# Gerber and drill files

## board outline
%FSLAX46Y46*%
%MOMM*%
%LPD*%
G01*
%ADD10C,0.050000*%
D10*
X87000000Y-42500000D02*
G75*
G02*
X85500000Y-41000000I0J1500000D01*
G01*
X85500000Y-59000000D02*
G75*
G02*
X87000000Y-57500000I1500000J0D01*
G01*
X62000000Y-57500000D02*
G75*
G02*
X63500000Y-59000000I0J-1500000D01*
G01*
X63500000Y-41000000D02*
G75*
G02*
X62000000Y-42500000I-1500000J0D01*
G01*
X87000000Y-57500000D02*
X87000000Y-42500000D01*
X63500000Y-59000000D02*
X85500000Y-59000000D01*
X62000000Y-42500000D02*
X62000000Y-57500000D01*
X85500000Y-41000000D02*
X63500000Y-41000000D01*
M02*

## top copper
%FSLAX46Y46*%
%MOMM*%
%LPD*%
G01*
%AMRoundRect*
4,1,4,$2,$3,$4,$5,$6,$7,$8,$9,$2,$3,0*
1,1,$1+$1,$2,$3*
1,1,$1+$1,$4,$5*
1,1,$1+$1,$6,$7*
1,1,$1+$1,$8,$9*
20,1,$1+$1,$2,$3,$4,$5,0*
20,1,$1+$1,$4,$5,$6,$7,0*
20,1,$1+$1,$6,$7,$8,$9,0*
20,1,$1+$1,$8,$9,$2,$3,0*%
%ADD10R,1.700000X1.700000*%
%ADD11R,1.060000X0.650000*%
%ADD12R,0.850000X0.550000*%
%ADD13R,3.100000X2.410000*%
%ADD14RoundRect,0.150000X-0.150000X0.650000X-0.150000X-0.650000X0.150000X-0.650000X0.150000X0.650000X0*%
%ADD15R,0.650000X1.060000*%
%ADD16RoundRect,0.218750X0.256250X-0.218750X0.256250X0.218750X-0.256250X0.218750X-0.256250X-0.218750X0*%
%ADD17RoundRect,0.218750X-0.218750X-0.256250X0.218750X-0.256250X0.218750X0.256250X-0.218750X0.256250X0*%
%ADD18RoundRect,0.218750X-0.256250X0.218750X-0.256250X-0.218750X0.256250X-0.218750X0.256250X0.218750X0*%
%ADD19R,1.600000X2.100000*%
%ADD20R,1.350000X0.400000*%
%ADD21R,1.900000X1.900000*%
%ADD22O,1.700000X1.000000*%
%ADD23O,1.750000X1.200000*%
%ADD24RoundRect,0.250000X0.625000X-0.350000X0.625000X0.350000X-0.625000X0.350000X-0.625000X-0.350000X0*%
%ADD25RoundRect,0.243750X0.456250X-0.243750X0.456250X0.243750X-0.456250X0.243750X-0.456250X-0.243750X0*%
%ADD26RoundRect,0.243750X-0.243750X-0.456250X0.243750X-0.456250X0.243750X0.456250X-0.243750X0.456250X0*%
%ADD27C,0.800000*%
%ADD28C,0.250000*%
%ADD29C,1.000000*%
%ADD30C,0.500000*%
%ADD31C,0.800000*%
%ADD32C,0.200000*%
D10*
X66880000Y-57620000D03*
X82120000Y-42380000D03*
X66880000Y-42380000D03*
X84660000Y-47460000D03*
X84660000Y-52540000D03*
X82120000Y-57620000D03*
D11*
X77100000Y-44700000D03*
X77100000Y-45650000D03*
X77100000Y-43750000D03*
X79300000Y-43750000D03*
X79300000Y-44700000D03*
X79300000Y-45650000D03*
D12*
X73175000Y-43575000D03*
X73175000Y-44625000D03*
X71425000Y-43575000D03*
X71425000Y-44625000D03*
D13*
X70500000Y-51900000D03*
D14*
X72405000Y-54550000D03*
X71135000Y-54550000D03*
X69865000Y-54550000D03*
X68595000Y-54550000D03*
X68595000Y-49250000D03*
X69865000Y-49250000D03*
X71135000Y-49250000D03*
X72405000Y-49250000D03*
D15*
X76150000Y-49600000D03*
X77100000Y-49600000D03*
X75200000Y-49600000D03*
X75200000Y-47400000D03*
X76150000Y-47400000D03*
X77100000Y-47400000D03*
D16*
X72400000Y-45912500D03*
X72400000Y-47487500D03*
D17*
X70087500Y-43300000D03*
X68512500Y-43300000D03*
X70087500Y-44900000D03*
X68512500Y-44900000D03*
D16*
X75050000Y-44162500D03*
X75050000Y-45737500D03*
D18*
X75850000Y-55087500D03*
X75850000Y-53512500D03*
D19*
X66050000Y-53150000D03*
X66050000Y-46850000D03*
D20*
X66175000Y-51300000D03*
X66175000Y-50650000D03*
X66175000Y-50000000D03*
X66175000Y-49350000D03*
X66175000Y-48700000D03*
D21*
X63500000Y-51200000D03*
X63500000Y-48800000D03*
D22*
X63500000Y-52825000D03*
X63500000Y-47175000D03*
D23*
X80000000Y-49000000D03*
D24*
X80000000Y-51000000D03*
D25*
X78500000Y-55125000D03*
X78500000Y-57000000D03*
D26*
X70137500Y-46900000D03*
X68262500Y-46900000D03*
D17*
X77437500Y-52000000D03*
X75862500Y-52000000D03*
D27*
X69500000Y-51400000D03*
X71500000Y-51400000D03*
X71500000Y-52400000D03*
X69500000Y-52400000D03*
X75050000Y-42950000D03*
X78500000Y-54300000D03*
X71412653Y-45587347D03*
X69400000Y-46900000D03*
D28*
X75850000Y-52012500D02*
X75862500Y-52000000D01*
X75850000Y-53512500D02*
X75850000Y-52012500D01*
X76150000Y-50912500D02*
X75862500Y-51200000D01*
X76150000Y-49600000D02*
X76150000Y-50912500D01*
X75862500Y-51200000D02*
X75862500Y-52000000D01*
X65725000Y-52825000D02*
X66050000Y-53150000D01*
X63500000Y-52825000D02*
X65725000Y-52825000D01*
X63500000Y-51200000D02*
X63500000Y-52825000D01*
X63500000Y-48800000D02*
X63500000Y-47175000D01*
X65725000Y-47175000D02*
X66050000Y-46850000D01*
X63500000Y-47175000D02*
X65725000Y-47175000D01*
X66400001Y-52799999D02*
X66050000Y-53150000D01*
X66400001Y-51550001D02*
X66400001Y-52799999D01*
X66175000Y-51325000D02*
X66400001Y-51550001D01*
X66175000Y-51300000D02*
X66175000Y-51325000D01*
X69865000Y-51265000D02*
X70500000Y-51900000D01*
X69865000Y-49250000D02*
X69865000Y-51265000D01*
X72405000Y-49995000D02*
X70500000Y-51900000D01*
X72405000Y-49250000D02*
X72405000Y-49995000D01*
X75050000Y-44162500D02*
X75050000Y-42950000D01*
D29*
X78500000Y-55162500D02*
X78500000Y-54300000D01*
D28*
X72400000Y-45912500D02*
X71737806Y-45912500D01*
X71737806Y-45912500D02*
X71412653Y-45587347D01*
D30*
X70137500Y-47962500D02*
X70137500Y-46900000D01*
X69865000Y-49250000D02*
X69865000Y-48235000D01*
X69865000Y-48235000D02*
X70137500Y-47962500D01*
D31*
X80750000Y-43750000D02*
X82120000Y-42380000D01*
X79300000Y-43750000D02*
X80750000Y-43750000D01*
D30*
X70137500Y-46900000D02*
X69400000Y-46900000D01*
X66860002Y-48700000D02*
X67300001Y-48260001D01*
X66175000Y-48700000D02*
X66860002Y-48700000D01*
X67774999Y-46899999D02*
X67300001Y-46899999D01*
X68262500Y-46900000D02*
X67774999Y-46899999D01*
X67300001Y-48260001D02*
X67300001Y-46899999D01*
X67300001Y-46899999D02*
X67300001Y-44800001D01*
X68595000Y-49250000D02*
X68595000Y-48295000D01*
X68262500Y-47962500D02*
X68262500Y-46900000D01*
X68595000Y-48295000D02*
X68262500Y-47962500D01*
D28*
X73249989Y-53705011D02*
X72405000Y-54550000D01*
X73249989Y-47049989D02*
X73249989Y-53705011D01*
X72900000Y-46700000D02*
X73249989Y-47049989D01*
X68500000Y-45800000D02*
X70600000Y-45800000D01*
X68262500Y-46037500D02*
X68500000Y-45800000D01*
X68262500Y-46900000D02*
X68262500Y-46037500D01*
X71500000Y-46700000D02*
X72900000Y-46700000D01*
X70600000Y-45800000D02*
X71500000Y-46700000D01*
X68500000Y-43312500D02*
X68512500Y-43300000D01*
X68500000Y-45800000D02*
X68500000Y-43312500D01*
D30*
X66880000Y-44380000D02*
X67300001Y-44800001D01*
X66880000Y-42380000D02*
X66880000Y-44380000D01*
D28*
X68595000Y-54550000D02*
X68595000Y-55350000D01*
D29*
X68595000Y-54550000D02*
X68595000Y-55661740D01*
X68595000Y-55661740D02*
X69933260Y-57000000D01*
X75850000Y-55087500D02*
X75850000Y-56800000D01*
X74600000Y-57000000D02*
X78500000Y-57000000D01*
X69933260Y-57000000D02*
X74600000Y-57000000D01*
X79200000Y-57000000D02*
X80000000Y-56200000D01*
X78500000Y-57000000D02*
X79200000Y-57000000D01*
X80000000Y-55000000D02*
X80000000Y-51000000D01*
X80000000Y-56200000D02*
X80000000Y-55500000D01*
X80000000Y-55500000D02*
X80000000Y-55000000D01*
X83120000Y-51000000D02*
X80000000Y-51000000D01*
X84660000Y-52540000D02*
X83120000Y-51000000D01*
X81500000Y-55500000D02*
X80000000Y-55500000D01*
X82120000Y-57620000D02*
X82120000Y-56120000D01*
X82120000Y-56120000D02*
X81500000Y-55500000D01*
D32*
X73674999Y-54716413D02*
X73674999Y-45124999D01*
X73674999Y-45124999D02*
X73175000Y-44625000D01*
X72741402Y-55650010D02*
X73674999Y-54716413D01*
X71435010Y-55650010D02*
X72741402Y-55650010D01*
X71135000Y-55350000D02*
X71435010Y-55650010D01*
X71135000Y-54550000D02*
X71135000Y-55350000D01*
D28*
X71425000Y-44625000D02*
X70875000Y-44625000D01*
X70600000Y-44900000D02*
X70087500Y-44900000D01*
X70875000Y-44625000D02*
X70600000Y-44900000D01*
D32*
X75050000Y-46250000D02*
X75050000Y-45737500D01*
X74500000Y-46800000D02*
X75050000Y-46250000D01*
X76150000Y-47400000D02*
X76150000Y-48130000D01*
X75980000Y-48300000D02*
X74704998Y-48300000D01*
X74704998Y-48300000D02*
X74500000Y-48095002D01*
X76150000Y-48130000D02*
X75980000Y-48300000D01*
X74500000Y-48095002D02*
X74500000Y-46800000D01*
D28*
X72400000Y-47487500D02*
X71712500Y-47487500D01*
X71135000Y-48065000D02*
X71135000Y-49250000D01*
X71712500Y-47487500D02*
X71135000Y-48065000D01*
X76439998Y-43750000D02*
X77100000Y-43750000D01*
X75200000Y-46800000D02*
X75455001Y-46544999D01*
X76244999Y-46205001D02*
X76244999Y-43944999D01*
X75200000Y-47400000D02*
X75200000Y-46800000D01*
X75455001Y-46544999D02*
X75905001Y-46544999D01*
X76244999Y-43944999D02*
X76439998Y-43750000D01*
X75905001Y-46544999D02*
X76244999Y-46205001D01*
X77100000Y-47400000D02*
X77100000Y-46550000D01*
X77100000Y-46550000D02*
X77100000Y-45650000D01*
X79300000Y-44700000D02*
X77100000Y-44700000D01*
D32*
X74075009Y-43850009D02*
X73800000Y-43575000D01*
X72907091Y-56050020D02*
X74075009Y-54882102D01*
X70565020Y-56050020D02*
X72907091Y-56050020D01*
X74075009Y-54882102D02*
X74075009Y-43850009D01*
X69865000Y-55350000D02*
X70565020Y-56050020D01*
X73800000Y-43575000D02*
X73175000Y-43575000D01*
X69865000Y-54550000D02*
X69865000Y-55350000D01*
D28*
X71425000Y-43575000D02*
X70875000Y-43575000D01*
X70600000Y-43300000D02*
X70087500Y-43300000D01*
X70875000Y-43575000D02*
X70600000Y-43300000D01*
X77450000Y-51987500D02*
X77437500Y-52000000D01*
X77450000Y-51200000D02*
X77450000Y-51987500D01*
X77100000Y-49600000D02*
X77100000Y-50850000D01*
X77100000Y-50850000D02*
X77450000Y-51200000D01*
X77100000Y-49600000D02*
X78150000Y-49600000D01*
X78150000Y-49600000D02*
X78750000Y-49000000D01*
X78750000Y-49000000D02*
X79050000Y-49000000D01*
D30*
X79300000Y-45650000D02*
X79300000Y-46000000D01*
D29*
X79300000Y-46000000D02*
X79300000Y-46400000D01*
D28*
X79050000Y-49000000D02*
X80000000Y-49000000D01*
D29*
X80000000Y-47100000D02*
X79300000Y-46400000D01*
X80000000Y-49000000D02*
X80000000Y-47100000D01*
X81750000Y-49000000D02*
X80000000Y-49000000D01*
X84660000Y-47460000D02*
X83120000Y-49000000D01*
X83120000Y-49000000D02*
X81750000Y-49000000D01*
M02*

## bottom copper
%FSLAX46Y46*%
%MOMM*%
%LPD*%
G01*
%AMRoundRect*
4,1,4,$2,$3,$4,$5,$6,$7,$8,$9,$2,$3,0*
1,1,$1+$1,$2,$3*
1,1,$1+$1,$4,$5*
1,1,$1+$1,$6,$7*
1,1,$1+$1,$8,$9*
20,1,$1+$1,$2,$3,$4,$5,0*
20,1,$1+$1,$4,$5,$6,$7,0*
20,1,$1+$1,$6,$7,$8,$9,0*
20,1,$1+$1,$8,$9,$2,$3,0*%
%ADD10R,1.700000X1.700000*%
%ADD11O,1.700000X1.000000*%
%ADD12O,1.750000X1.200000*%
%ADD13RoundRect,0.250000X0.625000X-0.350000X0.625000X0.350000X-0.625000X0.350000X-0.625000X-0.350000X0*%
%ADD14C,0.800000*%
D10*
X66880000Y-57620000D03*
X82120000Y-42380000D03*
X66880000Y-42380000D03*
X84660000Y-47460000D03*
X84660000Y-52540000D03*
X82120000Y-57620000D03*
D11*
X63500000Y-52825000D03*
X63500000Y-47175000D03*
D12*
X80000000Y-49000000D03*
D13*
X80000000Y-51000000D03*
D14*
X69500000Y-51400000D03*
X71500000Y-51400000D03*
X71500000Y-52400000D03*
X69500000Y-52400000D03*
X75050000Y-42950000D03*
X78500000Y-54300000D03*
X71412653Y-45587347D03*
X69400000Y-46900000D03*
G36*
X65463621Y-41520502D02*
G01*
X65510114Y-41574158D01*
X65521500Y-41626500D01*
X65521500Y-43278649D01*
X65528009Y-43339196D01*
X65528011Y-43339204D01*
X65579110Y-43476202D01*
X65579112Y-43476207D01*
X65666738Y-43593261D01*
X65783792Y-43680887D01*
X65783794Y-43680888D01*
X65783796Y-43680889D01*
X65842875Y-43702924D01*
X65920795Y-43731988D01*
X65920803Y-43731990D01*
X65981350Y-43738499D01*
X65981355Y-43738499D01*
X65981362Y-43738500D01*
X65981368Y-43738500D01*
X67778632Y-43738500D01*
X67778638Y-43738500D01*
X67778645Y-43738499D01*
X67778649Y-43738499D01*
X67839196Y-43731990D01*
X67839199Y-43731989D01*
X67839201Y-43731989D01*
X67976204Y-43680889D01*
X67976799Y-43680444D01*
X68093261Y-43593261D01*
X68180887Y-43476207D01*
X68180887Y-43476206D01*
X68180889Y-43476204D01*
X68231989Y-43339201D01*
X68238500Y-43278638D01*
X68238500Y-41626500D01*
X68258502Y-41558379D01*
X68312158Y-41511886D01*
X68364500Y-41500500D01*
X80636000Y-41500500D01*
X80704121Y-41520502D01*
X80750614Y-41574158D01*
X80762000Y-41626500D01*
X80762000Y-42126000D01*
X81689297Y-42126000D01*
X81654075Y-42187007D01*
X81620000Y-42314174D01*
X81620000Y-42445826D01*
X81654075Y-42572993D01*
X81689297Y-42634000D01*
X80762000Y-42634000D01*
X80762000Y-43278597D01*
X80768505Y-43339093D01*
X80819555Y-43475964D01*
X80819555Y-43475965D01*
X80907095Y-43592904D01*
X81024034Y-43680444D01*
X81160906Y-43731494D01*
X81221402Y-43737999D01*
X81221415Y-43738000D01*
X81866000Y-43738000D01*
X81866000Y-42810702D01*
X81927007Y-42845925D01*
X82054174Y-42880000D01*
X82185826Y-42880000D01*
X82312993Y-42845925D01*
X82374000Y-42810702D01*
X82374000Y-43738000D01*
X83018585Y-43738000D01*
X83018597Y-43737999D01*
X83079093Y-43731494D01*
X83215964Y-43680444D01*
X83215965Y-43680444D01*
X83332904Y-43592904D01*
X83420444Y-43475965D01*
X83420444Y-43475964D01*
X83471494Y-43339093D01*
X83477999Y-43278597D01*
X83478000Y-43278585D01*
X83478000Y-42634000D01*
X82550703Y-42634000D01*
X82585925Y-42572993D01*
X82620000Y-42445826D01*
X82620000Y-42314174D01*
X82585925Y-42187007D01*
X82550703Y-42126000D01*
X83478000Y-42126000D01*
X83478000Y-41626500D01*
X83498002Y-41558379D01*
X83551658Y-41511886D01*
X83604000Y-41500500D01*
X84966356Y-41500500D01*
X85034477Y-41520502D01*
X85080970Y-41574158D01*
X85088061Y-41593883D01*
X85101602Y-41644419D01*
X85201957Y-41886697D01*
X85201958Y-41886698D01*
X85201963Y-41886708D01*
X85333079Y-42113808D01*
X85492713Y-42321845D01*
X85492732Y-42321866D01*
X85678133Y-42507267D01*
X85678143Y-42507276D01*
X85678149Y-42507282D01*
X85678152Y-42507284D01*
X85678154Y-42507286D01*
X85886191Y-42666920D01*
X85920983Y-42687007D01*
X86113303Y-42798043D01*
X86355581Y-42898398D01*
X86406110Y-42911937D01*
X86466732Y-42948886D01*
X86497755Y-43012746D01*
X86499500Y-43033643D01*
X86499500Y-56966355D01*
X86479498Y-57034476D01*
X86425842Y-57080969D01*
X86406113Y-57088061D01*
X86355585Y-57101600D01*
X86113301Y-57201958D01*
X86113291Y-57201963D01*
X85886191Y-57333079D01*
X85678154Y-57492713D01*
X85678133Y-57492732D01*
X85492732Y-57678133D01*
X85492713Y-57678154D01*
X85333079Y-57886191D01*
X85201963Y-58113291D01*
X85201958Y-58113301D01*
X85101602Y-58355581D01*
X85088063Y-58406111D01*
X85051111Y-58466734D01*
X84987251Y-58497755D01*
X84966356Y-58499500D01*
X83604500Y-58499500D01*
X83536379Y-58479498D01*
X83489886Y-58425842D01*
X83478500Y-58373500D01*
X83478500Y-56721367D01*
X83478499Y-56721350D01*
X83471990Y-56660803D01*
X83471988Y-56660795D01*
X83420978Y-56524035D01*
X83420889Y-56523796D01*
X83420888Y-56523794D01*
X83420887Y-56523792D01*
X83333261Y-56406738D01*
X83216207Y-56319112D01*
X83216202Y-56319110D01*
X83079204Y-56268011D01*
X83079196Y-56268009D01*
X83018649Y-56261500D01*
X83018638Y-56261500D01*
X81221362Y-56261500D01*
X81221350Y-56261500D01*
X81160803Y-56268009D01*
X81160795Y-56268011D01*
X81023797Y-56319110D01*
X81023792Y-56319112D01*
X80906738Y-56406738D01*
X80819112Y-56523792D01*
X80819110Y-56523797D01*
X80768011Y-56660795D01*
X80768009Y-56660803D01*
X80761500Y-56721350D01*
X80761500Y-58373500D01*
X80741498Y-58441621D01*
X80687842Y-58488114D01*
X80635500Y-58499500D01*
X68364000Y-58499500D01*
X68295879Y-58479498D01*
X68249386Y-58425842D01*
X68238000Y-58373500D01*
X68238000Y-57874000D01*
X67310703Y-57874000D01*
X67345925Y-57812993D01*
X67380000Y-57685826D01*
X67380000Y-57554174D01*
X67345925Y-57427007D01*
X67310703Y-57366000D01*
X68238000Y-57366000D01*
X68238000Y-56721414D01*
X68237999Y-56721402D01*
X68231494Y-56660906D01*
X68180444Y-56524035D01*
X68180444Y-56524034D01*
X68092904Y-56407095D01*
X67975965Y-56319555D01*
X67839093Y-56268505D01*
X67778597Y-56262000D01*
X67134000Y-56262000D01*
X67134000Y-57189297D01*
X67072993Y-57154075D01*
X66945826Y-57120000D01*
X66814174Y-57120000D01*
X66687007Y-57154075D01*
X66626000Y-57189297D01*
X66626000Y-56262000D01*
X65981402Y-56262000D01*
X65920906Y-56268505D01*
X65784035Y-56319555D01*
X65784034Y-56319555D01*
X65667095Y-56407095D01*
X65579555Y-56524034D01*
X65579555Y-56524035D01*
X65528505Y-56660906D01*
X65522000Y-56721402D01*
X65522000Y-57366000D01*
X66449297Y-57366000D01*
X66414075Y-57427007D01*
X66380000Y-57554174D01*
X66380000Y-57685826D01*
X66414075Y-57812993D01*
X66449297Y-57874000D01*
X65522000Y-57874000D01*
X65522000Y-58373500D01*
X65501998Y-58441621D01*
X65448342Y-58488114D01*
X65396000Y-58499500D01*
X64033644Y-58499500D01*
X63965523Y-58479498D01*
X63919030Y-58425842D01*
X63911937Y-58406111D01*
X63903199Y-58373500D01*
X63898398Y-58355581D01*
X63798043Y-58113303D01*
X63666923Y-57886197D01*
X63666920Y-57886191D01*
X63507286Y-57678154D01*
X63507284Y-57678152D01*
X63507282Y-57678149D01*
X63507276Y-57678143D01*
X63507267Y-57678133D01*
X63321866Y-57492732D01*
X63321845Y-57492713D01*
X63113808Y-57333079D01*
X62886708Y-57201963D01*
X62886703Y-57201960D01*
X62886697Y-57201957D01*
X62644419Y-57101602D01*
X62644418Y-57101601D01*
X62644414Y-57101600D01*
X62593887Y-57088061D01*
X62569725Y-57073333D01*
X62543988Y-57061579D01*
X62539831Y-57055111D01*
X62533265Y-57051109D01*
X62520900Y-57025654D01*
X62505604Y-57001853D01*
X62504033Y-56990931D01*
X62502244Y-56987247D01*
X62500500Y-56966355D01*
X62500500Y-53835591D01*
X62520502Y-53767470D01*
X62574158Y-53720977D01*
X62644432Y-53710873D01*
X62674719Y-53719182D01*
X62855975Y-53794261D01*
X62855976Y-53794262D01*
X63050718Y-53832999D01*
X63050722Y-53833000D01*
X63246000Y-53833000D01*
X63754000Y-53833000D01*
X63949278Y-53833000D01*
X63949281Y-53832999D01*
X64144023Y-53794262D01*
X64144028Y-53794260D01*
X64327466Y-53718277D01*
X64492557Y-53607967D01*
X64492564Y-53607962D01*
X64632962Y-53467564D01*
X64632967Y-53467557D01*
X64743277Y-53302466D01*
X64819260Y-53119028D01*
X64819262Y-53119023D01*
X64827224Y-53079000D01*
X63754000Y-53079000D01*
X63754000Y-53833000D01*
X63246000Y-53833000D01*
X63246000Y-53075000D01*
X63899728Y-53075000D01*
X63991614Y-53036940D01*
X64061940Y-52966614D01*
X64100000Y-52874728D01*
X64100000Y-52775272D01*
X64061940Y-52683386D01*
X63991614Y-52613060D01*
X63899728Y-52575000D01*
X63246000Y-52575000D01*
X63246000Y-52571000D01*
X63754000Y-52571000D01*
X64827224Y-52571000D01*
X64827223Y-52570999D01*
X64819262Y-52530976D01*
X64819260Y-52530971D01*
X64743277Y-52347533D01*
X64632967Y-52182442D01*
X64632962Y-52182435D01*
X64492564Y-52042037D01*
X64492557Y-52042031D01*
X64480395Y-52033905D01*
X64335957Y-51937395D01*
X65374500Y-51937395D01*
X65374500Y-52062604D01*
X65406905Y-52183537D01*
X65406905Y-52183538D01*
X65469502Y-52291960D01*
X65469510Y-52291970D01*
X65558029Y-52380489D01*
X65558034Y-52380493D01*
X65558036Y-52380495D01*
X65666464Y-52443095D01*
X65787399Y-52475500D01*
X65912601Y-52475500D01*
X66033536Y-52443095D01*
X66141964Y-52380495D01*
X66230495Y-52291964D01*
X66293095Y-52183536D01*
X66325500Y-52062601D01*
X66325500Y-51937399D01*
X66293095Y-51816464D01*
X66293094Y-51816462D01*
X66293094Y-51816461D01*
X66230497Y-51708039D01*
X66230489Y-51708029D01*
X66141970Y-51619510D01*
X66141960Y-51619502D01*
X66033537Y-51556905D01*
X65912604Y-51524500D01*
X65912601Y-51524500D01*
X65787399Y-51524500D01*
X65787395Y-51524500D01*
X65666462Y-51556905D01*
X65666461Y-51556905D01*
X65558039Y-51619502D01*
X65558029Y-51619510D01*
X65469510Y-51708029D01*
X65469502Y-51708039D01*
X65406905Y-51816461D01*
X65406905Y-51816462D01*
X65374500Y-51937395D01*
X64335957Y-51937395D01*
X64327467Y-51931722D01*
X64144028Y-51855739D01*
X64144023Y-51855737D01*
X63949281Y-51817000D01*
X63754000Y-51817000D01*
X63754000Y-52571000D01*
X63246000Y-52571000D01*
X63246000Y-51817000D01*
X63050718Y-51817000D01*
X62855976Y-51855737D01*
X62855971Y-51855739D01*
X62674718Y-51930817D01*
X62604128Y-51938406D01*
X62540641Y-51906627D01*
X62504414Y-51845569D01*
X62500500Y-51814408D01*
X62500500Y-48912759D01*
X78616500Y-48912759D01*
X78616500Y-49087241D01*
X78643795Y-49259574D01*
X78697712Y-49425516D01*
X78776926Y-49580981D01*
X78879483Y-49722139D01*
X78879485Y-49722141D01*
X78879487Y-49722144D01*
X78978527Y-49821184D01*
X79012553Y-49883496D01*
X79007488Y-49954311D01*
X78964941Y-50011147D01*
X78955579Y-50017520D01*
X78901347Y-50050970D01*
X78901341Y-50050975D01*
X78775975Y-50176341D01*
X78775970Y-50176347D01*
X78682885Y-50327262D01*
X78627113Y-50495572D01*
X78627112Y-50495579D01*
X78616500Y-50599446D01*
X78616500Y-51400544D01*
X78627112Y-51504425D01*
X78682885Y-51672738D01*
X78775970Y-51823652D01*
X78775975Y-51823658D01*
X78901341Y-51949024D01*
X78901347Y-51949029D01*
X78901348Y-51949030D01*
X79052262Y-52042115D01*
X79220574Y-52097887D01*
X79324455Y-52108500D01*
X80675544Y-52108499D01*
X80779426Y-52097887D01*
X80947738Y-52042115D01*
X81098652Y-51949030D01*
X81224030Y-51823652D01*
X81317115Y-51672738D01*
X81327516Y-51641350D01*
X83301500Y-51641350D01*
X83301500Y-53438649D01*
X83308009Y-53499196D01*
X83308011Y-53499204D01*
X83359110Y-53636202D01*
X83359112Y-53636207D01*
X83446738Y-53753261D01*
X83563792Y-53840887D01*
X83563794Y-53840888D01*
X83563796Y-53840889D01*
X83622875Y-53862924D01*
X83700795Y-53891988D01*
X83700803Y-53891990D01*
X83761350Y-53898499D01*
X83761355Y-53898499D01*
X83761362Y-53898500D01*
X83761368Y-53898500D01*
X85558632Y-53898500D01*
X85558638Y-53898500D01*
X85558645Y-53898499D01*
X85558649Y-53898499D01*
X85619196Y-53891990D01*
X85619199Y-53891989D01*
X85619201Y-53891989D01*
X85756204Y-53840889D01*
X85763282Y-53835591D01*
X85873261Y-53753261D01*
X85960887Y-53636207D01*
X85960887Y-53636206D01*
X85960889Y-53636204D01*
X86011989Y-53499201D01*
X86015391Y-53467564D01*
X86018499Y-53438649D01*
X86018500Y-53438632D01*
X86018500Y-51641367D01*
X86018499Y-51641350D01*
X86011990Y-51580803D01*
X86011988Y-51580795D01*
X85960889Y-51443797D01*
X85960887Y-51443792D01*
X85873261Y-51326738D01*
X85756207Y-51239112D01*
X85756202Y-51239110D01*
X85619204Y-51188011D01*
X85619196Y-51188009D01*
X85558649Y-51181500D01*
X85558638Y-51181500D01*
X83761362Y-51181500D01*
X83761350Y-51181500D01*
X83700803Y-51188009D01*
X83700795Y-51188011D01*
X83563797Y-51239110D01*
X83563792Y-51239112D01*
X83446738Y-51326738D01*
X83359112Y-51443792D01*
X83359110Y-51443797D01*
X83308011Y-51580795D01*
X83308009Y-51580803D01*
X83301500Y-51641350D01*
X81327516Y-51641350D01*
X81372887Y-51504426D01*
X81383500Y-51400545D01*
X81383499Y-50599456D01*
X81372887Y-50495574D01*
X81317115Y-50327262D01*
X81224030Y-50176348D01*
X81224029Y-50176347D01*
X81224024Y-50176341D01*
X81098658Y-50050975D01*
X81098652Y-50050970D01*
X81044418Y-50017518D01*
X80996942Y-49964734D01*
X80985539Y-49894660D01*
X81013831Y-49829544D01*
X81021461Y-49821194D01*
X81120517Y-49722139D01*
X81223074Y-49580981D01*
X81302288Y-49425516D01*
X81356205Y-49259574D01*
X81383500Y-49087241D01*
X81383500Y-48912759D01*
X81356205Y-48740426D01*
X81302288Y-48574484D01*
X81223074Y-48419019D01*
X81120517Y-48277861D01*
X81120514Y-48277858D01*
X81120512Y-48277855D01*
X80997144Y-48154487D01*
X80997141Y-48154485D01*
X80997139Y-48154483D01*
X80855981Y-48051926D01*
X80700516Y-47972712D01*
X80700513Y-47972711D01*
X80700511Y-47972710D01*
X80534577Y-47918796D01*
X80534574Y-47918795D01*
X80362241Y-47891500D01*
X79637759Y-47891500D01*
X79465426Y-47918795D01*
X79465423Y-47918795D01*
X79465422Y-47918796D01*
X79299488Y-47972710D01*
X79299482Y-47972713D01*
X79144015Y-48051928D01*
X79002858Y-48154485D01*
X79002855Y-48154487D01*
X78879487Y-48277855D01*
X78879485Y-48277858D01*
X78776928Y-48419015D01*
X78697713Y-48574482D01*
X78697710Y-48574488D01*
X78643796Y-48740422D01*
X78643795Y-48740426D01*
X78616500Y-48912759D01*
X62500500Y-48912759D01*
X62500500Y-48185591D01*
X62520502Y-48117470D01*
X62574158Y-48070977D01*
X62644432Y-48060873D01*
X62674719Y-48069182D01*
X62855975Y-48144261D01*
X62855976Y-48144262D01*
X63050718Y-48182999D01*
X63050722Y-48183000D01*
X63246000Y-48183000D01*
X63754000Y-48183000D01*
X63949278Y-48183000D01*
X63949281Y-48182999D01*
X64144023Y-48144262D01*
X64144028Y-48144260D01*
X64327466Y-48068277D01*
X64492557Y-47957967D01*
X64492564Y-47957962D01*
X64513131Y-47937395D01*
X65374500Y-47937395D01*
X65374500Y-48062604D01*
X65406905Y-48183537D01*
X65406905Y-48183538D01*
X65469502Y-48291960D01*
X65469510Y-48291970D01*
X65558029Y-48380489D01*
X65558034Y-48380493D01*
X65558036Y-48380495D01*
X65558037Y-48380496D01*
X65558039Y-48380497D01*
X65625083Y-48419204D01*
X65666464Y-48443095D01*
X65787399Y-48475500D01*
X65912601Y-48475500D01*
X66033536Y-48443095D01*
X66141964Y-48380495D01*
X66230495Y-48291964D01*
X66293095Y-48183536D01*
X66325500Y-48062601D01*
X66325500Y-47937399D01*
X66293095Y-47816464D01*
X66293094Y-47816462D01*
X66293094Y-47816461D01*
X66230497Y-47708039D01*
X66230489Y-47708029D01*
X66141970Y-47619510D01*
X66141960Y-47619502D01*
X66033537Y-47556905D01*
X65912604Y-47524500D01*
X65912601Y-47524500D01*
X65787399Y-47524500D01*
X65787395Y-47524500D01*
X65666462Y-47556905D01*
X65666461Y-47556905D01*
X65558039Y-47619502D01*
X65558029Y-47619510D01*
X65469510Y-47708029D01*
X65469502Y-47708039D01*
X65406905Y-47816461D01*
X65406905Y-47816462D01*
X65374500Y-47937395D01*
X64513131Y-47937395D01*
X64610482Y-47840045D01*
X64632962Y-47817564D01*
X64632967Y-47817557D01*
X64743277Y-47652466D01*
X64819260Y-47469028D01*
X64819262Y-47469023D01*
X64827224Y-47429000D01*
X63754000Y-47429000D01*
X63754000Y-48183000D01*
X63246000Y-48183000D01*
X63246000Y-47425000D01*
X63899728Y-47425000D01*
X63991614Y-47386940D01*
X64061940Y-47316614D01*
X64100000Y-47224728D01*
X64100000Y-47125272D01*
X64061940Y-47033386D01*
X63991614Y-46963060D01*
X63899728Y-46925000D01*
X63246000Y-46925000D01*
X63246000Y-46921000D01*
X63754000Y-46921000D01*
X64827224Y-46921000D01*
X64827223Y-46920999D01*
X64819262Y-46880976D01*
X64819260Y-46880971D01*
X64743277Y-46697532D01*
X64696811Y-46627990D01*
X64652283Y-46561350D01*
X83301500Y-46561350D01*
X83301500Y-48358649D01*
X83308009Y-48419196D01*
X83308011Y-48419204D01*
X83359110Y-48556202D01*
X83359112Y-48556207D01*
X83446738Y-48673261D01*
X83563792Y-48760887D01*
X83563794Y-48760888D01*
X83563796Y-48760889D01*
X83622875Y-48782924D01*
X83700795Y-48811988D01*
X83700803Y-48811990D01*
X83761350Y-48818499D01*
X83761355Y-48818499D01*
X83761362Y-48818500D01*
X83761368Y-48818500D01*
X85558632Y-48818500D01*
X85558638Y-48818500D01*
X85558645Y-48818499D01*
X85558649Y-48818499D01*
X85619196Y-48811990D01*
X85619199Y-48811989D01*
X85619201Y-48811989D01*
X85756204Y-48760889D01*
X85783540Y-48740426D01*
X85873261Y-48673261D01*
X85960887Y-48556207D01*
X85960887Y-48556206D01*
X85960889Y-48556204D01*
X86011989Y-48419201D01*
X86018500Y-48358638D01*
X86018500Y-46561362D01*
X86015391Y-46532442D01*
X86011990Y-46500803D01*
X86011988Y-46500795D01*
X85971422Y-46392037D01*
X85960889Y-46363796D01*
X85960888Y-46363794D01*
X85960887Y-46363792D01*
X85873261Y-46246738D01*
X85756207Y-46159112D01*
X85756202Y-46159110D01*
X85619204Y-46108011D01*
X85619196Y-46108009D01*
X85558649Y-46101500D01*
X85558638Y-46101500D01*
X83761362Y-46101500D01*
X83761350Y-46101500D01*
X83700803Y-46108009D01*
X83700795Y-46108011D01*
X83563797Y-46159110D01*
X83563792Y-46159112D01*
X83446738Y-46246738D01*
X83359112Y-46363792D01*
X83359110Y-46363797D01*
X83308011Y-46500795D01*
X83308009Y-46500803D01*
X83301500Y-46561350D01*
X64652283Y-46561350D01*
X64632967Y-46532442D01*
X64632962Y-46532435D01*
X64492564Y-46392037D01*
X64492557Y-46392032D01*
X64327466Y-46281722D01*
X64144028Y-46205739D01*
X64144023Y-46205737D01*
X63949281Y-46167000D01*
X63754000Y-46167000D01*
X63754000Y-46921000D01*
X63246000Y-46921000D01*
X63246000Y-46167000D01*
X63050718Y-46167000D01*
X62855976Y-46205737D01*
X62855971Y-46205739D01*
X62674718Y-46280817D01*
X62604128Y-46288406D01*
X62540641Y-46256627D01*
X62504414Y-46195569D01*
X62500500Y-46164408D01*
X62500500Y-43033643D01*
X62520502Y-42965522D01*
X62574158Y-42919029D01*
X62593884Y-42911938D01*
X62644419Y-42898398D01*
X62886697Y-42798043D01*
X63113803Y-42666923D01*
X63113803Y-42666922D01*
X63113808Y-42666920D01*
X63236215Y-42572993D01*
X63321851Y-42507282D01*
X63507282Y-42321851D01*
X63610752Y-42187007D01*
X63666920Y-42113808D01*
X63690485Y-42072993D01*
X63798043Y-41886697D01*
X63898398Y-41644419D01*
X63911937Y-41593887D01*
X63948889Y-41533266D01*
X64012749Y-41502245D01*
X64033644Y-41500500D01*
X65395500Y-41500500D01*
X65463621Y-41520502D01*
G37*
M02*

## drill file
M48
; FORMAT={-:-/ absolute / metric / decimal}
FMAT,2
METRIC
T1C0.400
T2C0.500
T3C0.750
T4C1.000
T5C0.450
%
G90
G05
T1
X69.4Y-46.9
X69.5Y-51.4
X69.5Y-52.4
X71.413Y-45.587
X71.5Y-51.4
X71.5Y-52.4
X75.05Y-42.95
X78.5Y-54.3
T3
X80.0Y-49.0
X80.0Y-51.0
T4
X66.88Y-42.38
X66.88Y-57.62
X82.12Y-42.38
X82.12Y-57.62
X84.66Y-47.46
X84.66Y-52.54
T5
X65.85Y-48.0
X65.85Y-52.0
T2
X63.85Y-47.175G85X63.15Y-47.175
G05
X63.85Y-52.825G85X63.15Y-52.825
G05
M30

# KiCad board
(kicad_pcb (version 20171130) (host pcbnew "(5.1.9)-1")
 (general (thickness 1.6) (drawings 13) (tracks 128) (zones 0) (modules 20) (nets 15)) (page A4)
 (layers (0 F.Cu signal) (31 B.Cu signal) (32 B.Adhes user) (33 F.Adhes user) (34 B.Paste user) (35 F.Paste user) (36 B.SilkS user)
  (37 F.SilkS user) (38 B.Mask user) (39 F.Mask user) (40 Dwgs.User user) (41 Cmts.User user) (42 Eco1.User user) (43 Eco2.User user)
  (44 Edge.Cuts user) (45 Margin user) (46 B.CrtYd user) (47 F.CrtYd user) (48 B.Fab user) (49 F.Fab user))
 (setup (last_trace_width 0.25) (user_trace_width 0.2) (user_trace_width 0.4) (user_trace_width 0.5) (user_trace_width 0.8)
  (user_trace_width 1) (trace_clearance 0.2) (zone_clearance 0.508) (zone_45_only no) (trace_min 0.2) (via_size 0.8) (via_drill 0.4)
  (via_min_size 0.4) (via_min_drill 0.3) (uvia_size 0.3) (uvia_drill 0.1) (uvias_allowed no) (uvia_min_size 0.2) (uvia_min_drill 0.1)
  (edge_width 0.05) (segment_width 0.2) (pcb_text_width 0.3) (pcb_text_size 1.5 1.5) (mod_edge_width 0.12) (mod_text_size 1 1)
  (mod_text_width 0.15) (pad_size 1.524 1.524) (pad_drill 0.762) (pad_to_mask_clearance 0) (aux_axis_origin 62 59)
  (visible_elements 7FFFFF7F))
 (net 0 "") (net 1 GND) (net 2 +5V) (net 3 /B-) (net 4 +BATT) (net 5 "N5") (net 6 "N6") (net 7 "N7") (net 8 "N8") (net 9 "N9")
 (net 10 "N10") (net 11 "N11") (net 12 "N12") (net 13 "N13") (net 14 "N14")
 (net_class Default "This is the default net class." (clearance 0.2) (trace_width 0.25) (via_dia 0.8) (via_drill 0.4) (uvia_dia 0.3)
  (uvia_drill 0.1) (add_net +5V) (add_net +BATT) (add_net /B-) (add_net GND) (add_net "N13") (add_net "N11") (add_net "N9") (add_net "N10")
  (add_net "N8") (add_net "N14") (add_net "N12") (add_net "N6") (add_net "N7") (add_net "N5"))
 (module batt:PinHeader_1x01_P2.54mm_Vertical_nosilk (layer F.Cu) (at 66.88 57.62 90)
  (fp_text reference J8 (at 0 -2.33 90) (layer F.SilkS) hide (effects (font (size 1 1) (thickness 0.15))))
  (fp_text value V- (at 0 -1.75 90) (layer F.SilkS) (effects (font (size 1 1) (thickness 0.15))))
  (pad 1 thru_hole rect (at 0 0 90) (size 1.7 1.7) (drill 1) (layers *.Cu *.Mask) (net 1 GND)))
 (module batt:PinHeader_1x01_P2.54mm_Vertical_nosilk (layer F.Cu) (at 82.12 42.38 270)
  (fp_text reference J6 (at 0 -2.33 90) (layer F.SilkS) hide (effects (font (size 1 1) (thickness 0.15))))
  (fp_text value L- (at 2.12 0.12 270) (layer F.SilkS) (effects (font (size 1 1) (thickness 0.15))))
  (pad 1 thru_hole rect (at 0 0 270) (size 1.7 1.7) (drill 1) (layers *.Cu *.Mask) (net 1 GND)))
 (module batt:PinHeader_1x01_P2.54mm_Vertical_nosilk (layer F.Cu) (at 66.88 42.38 180)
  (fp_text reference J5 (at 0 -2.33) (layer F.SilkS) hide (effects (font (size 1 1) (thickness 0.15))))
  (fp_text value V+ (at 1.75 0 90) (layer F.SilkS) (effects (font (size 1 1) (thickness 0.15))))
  (pad 1 thru_hole rect (at 0 0 180) (size 1.7 1.7) (drill 1) (layers *.Cu *.Mask) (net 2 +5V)))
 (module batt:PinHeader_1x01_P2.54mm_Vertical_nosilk (layer F.Cu) (at 84.66 47.46)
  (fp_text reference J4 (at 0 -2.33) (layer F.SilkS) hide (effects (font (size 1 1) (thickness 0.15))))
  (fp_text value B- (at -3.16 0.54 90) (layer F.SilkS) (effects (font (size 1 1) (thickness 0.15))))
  (pad 1 thru_hole rect (at 0 0) (size 1.7 1.7) (drill 1) (layers *.Cu *.Mask) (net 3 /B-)))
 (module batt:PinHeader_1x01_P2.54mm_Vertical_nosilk (layer F.Cu) (at 84.66 52.54 180)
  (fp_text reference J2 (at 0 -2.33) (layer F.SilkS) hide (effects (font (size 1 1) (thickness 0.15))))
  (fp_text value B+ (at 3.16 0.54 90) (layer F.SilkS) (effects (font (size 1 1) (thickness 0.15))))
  (pad 1 thru_hole rect (at 0 0 180) (size 1.7 1.7) (drill 1) (layers *.Cu *.Mask) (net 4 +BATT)))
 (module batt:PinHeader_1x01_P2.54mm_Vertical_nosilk (layer F.Cu) (at 82.12 57.62)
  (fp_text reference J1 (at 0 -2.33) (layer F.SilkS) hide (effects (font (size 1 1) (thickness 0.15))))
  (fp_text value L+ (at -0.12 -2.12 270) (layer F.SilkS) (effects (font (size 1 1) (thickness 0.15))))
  (pad 1 thru_hole rect (at 0 0) (size 1.7 1.7) (drill 1) (layers *.Cu *.Mask) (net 4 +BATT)))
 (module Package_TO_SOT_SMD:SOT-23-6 (layer F.Cu) (at 78.2 44.7 180)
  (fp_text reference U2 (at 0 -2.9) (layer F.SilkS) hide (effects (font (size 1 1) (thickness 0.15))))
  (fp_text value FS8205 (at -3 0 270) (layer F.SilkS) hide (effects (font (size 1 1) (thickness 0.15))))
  (pad 5 smd rect (at 1.1 0 180) (size 1.06 0.65) (layers F.Cu F.Paste F.Mask) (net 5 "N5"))
  (pad 6 smd rect (at 1.1 -0.95 180) (size 1.06 0.65) (layers F.Cu F.Paste F.Mask) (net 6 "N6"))
  (pad 4 smd rect (at 1.1 0.95 180) (size 1.06 0.65) (layers F.Cu F.Paste F.Mask) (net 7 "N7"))
  (pad 3 smd rect (at -1.1 0.95 180) (size 1.06 0.65) (layers F.Cu F.Paste F.Mask) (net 1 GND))
  (pad 2 smd rect (at -1.1 0 180) (size 1.06 0.65) (layers F.Cu F.Paste F.Mask) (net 5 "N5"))
  (pad 1 smd rect (at -1.1 -0.95 180) (size 1.06 0.65) (layers F.Cu F.Paste F.Mask) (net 3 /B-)))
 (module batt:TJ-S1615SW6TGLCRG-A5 (layer F.Cu) (at 72.3 44.1 180)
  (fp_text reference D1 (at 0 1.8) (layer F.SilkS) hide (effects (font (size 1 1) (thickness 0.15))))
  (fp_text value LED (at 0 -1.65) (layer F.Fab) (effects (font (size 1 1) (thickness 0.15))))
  (pad 4 smd rect (at -0.875 0.525 180) (size 0.85 0.55) (layers F.Cu F.Paste F.Mask) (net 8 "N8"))
  (pad 2 smd rect (at -0.875 -0.525 180) (size 0.85 0.55) (layers F.Cu F.Paste F.Mask) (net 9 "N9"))
  (pad 3 smd rect (at 0.875 0.525 180) (size 0.85 0.55) (layers F.Cu F.Paste F.Mask) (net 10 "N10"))
  (pad 1 smd rect (at 0.875 -0.525 180) (size 0.85 0.55) (layers F.Cu F.Paste F.Mask) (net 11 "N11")))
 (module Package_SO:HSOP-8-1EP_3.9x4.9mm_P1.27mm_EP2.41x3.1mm (layer F.Cu) (at 70.5 51.9 270)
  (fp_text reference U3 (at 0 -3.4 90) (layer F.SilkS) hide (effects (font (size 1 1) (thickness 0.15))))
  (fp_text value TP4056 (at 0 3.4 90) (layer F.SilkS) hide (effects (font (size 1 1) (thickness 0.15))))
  (pad "" smd roundrect (at 0.6 0.775 270) (size 0.97 1.25) (layers F.Paste) (roundrect_rratio 0.25))
  (pad "" smd roundrect (at 0.6 -0.775 270) (size 0.97 1.25) (layers F.Paste) (roundrect_rratio 0.25))
  (pad "" smd roundrect (at -0.6 0.775 270) (size 0.97 1.25) (layers F.Paste) (roundrect_rratio 0.25))
  (pad "" smd roundrect (at -0.6 -0.775 270) (size 0.97 1.25) (layers F.Paste) (roundrect_rratio 0.25))
  (pad 9 smd rect (at 0 0 270) (size 2.41 3.1) (layers F.Cu F.Mask) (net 1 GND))
  (pad 8 smd roundrect (at 2.65 -1.905 270) (size 1.6 0.6) (layers F.Cu F.Paste F.Mask) (roundrect_rratio 0.25) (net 2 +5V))
  (pad 7 smd roundrect (at 2.65 -0.635 270) (size 1.6 0.6) (layers F.Cu F.Paste F.Mask) (roundrect_rratio 0.25) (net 9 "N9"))
  (pad 6 smd roundrect (at 2.65 0.635 270) (size 1.6 0.6) (layers F.Cu F.Paste F.Mask) (roundrect_rratio 0.25) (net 8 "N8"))
  (pad 5 smd roundrect (at 2.65 1.905 270) (size 1.6 0.6) (layers F.Cu F.Paste F.Mask) (roundrect_rratio 0.25) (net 4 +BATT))
  (pad 4 smd roundrect (at -2.65 1.905 270) (size 1.6 0.6) (layers F.Cu F.Paste F.Mask) (roundrect_rratio 0.25) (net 2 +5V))
  (pad 3 smd roundrect (at -2.65 0.635 270) (size 1.6 0.6) (layers F.Cu F.Paste F.Mask) (roundrect_rratio 0.25) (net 1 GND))
  (pad 2 smd roundrect (at -2.65 -0.635 270) (size 1.6 0.6) (layers F.Cu F.Paste F.Mask) (roundrect_rratio 0.25) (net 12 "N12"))
  (pad 1 smd roundrect (at -2.65 -1.905 270) (size 1.6 0.6) (layers F.Cu F.Paste F.Mask) (roundrect_rratio 0.25) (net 1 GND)))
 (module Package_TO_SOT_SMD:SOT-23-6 (layer F.Cu) (at 76.15 48.5 270)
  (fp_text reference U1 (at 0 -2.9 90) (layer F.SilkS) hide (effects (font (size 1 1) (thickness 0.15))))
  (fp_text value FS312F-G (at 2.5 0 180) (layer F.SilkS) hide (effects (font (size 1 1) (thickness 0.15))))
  (pad 5 smd rect (at 1.1 0 270) (size 1.06 0.65) (layers F.Cu F.Paste F.Mask) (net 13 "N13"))
  (pad 6 smd rect (at 1.1 -0.95 270) (size 1.06 0.65) (layers F.Cu F.Paste F.Mask) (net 3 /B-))
  (pad 4 smd rect (at 1.1 0.95 270) (size 1.06 0.65) (layers F.Cu F.Paste F.Mask))
  (pad 3 smd rect (at -1.1 0.95 270) (size 1.06 0.65) (layers F.Cu F.Paste F.Mask) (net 7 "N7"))
  (pad 2 smd rect (at -1.1 0 270) (size 1.06 0.65) (layers F.Cu F.Paste F.Mask) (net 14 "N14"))
  (pad 1 smd rect (at -1.1 -0.95 270) (size 1.06 0.65) (layers F.Cu F.Paste F.Mask) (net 6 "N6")))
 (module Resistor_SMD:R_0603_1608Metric (layer F.Cu) (at 72.4 46.7 90)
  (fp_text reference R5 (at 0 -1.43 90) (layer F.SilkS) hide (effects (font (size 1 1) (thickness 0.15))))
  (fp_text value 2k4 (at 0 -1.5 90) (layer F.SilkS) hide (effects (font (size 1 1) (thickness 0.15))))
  (pad 2 smd roundrect (at 0.7875 0 90) (size 0.875 0.95) (layers F.Cu F.Paste F.Mask) (roundrect_rratio 0.25) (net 1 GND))
  (pad 1 smd roundrect (at -0.7875 0 90) (size 0.875 0.95) (layers F.Cu F.Paste F.Mask) (roundrect_rratio 0.25) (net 12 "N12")))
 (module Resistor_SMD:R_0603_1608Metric (layer F.Cu) (at 69.3 43.3)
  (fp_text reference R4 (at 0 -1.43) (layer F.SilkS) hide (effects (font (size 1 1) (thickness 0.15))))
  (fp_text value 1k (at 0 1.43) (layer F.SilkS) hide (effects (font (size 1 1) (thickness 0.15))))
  (pad 2 smd roundrect (at 0.7875 0) (size 0.875 0.95) (layers F.Cu F.Paste F.Mask) (roundrect_rratio 0.25) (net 10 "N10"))
  (pad 1 smd roundrect (at -0.7875 0) (size 0.875 0.95) (layers F.Cu F.Paste F.Mask) (roundrect_rratio 0.25) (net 2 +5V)))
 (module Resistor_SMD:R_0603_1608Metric (layer F.Cu) (at 69.3 44.9)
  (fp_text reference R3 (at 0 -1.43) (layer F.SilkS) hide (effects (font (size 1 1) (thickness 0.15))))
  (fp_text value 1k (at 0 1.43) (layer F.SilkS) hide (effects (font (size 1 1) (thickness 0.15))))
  (pad 2 smd roundrect (at 0.7875 0) (size 0.875 0.95) (layers F.Cu F.Paste F.Mask) (roundrect_rratio 0.25) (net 11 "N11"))
  (pad 1 smd roundrect (at -0.7875 0) (size 0.875 0.95) (layers F.Cu F.Paste F.Mask) (roundrect_rratio 0.25) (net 2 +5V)))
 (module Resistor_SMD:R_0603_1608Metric (layer F.Cu) (at 75.05 44.95 90)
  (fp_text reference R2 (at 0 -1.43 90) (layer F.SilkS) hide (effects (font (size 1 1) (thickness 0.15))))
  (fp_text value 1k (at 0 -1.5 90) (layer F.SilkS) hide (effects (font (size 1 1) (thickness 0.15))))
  (pad 2 smd roundrect (at 0.7875 0 90) (size 0.875 0.95) (layers F.Cu F.Paste F.Mask) (roundrect_rratio 0.25) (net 1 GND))
  (pad 1 smd roundrect (at -0.7875 0 90) (size 0.875 0.95) (layers F.Cu F.Paste F.Mask) (roundrect_rratio 0.25) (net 14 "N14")))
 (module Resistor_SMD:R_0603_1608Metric (layer F.Cu) (at 75.85 54.3 270)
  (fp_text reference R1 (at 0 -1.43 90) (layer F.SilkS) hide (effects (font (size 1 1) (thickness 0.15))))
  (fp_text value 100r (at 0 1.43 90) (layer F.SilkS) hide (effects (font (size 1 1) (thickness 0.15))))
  (pad 2 smd roundrect (at 0.7875 0 270) (size 0.875 0.95) (layers F.Cu F.Paste F.Mask) (roundrect_rratio 0.25) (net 4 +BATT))
  (pad 1 smd roundrect (at -0.7875 0 270) (size 0.875 0.95) (layers F.Cu F.Paste F.Mask) (roundrect_rratio 0.25) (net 13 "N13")))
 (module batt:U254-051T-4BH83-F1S (layer F.Cu) (at 63.5 50 270)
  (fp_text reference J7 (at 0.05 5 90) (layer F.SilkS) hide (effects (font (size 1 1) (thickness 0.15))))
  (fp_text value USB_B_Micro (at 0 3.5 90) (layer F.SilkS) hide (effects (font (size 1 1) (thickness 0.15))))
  (pad 6 smd rect (at 3.15 -2.55 270) (size 2.1 1.6) (layers F.Cu F.Paste F.Mask) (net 1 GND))
  (pad 6 smd rect (at -3.15 -2.55 270) (size 2.1 1.6) (layers F.Cu F.Paste F.Mask) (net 1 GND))
  (pad 5 smd rect (at 1.3 -2.675 270) (size 0.4 1.35) (layers F.Cu F.Paste F.Mask) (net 1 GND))
  (pad 4 smd rect (at 0.65 -2.675 270) (size 0.4 1.35) (layers F.Cu F.Paste F.Mask))
  (pad 3 smd rect (at 0 -2.675 270) (size 0.4 1.35) (layers F.Cu F.Paste F.Mask))
  (pad 2 smd rect (at -0.65 -2.675 270) (size 0.4 1.35) (layers F.Cu F.Paste F.Mask))
  (pad 1 smd rect (at -1.3 -2.675 270) (size 0.4 1.35) (layers F.Cu F.Paste F.Mask) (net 2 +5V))
  (pad "" np_thru_hole circle (at 2 -2.35 270) (size 0.45 0.45) (drill 0.45) (layers *.Cu *.Mask))
  (pad "" np_thru_hole circle (at -2 -2.35 270) (size 0.45 0.45) (drill 0.45) (layers *.Cu *.Mask))
  (pad 6 smd rect (at 1.2 0 270) (size 1.9 1.9) (layers F.Cu F.Paste F.Mask) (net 1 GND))
  (pad 6 smd rect (at -1.2 0 270) (size 1.9 1.9) (layers F.Cu F.Paste F.Mask) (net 1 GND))
  (pad 6 thru_hole oval (at 2.825 0 270) (size 1 1.7) (drill oval 0.5 1.2) (layers *.Cu *.Mask) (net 1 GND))
  (pad 6 thru_hole oval (at -2.825 0 270) (size 1 1.7) (drill oval 0.5 1.2) (layers *.Cu *.Mask) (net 1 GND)))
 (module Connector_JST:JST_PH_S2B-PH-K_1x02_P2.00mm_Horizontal (layer F.Cu) (at 80 51 90)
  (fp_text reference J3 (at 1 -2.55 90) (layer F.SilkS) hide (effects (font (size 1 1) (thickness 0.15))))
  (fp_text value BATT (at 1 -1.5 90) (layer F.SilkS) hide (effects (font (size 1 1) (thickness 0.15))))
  (pad 2 thru_hole oval (at 2 0 90) (size 1.2 1.75) (drill 0.75) (layers *.Cu *.Mask) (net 3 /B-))
  (pad 1 thru_hole roundrect (at 0 0 90) (size 1.2 1.75) (drill 0.75) (layers *.Cu *.Mask) (roundrect_rratio 0.208333) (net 4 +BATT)))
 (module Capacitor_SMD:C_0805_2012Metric (layer F.Cu) (at 78.5 56.0625 90)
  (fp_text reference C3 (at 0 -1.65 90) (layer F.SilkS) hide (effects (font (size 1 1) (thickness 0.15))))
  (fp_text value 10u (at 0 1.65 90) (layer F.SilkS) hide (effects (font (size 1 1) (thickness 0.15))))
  (pad 2 smd roundrect (at 0.9375 0 90) (size 0.975 1.4) (layers F.Cu F.Paste F.Mask) (roundrect_rratio 0.25) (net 1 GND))
  (pad 1 smd roundrect (at -0.9375 0 90) (size 0.975 1.4) (layers F.Cu F.Paste F.Mask) (roundrect_rratio 0.25) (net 4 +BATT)))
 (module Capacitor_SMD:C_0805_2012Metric (layer F.Cu) (at 69.2 46.9)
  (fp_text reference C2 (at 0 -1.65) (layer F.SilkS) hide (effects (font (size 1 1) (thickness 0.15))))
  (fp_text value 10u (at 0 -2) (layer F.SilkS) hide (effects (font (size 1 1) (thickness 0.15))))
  (pad 2 smd roundrect (at 0.9375 0) (size 0.975 1.4) (layers F.Cu F.Paste F.Mask) (roundrect_rratio 0.25) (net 1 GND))
  (pad 1 smd roundrect (at -0.9375 0) (size 0.975 1.4) (layers F.Cu F.Paste F.Mask) (roundrect_rratio 0.25) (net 2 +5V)))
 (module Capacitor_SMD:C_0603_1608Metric (layer F.Cu) (at 76.65 52)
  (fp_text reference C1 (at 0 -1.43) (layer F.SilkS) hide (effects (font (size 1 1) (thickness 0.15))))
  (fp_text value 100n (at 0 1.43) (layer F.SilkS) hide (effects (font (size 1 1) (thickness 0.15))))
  (pad 2 smd roundrect (at 0.7875 0) (size 0.875 0.95) (layers F.Cu F.Paste F.Mask) (roundrect_rratio 0.25) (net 3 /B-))
  (pad 1 smd roundrect (at -0.7875 0) (size 0.875 0.95) (layers F.Cu F.Paste F.Mask) (roundrect_rratio 0.25) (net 13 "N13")))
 (gr_arc (start 87 41) (end 85.5 41) (angle -90) (layer Edge.Cuts) (width 0.05))
 (gr_arc (start 87 59) (end 87 57.5) (angle -90) (layer Edge.Cuts) (width 0.05))
 (gr_arc (start 62 59) (end 63.5 59) (angle -90) (layer Edge.Cuts) (width 0.05))
 (gr_arc (start 62 41) (end 62 42.5) (angle -90) (layer Edge.Cuts) (width 0.05))
 (gr_line (start 87 57.5) (end 87 42.5) (layer Edge.Cuts) (width 0.05))
 (gr_line (start 63.5 59) (end 85.5 59) (layer Edge.Cuts) (width 0.05))
 (gr_line (start 62 42.5) (end 62 57.5) (layer Edge.Cuts) (width 0.05))
 (gr_line (start 85.5 41) (end 63.5 41) (layer Edge.Cuts) (width 0.05))
 (segment (start 75.85 52.0125) (end 75.8625 52) (width 0.25) (layer F.Cu) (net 13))
 (segment (start 75.85 53.5125) (end 75.85 52.0125) (width 0.25) (layer F.Cu) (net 13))
 (segment (start 76.15 50.9125) (end 75.8625 51.2) (width 0.25) (layer F.Cu) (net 13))
 (segment (start 76.15 49.6) (end 76.15 50.9125) (width 0.25) (layer F.Cu) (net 13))
 (segment (start 75.8625 51.2) (end 75.8625 52) (width 0.25) (layer F.Cu) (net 13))
 (via (at 69.5 51.4) (size 0.8) (drill 0.4) (layers F.Cu B.Cu) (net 1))
 (via (at 71.5 51.4) (size 0.8) (drill 0.4) (layers F.Cu B.Cu) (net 1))
 (via (at 71.5 52.4) (size 0.8) (drill 0.4) (layers F.Cu B.Cu) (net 1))
 (via (at 69.5 52.4) (size 0.8) (drill 0.4) (layers F.Cu B.Cu) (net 1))
 (segment (start 65.725 52.825) (end 66.05 53.15) (width 0.25) (layer F.Cu) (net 1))
 (segment (start 63.5 52.825) (end 65.725 52.825) (width 0.25) (layer F.Cu) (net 1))
 (segment (start 63.5 51.2) (end 63.5 52.825) (width 0.25) (layer F.Cu) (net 1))
 (segment (start 63.5 48.8) (end 63.5 47.175) (width 0.25) (layer F.Cu) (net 1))
 (segment (start 65.725 47.175) (end 66.05 46.85) (width 0.25) (layer F.Cu) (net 1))
 (segment (start 63.5 47.175) (end 65.725 47.175) (width 0.25) (layer F.Cu) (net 1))
 (segment (start 66.400001 52.799999) (end 66.05 53.15) (width 0.25) (layer F.Cu) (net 1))
 (segment (start 66.400001 51.550001) (end 66.400001 52.799999) (width 0.25) (layer F.Cu) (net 1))
 (segment (start 66.175 51.325) (end 66.400001 51.550001) (width 0.25) (layer F.Cu) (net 1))
 (segment (start 66.175 51.3) (end 66.175 51.325) (width 0.25) (layer F.Cu) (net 1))
 (segment (start 69.865 51.265) (end 70.5 51.9) (width 0.25) (layer F.Cu) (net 1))
 (segment (start 69.865 49.25) (end 69.865 51.265) (width 0.25) (layer F.Cu) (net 1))
 (segment (start 72.405 49.995) (end 70.5 51.9) (width 0.25) (layer F.Cu) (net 1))
 (segment (start 72.405 49.25) (end 72.405 49.995) (width 0.25) (layer F.Cu) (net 1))
 (via (at 75.05 42.95) (size 0.8) (drill 0.4) (layers F.Cu B.Cu) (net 1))
 (segment (start 75.05 44.1625) (end 75.05 42.95) (width 0.25) (layer F.Cu) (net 1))
 (via (at 78.5 54.3) (size 0.8) (drill 0.4) (layers F.Cu B.Cu) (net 1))
 (segment (start 78.5 55.1625) (end 78.5 54.3) (width 1) (layer F.Cu) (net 1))
 (segment (start 72.4 45.9125) (end 71.737806 45.9125) (width 0.25) (layer F.Cu) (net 1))
 (via (at 71.412653 45.587347) (size 0.8) (drill 0.4) (layers F.Cu B.Cu) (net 1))
 (segment (start 71.737806 45.9125) (end 71.412653 45.587347) (width 0.25) (layer F.Cu) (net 1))
 (segment (start 70.1375 47.9625) (end 70.1375 46.9) (width 0.5) (layer F.Cu) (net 1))
 (segment (start 69.865 49.25) (end 69.865 48.235) (width 0.5) (layer F.Cu) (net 1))
 (segment (start 69.865 48.235) (end 70.1375 47.9625) (width 0.5) (layer F.Cu) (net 1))
 (segment (start 80.75 43.75) (end 82.12 42.38) (width 0.8) (layer F.Cu) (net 1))
 (segment (start 79.3 43.75) (end 80.75 43.75) (width 0.8) (layer F.Cu) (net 1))
 (via (at 69.4 46.9) (size 0.8) (drill 0.4) (layers F.Cu B.Cu) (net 1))
 (segment (start 70.1375 46.9) (end 69.4 46.9) (width 0.5) (layer F.Cu) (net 1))
 (segment (start 66.860002 48.7) (end 67.300001 48.260001) (width 0.5) (layer F.Cu) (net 2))
 (segment (start 66.175 48.7) (end 66.860002 48.7) (width 0.5) (layer F.Cu) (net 2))
 (segment (start 67.774999 46.899999) (end 67.300001 46.899999) (width 0.5) (layer F.Cu) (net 2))
 (segment (start 68.2625 46.9) (end 67.774999 46.899999) (width 0.5) (layer F.Cu) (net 2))
 (segment (start 67.300001 48.260001) (end 67.300001 46.899999) (width 0.5) (layer F.Cu) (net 2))
 (segment (start 67.300001 46.899999) (end 67.300001 44.800001) (width 0.5) (layer F.Cu) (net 2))
 (segment (start 68.595 49.25) (end 68.595 48.295) (width 0.5) (layer F.Cu) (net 2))
 (segment (start 68.2625 47.9625) (end 68.2625 46.9) (width 0.5) (layer F.Cu) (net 2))
 (segment (start 68.595 48.295) (end 68.2625 47.9625) (width 0.5) (layer F.Cu) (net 2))
 (segment (start 73.249989 53.705011) (end 72.405 54.55) (width 0.25) (layer F.Cu) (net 2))
 (segment (start 73.249989 47.049989) (end 73.249989 53.705011) (width 0.25) (layer F.Cu) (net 2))
 (segment (start 72.9 46.7) (end 73.249989 47.049989) (width 0.25) (layer F.Cu) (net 2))
 (segment (start 68.5 45.8) (end 70.6 45.8) (width 0.25) (layer F.Cu) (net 2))
 (segment (start 68.2625 46.0375) (end 68.5 45.8) (width 0.25) (layer F.Cu) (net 2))
 (segment (start 68.2625 46.9) (end 68.2625 46.0375) (width 0.25) (layer F.Cu) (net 2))
 (segment (start 71.5 46.7) (end 72.9 46.7) (width 0.25) (layer F.Cu) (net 2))
 (segment (start 70.6 45.8) (end 71.5 46.7) (width 0.25) (layer F.Cu) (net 2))
 (segment (start 68.5 43.3125) (end 68.5125 43.3) (width 0.25) (layer F.Cu) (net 2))
 (segment (start 68.5 45.8) (end 68.5 43.3125) (width 0.25) (layer F.Cu) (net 2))
 (segment (start 66.88 44.38) (end 67.300001 44.800001) (width 0.5) (layer F.Cu) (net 2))
 (segment (start 66.88 42.38) (end 66.88 44.38) (width 0.5) (layer F.Cu) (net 2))
 (segment (start 68.595 54.55) (end 68.595 55.35) (width 0.25) (layer F.Cu) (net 4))
 (segment (start 68.595 54.55) (end 68.595 55.66174) (width 1) (layer F.Cu) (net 4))
 (segment (start 68.595 55.66174) (end 69.93326 57) (width 1) (layer F.Cu) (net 4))
 (segment (start 75.85 55.0875) (end 75.85 56.8) (width 1) (layer F.Cu) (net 4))
 (segment (start 74.6 57) (end 78.5 57) (width 1) (layer F.Cu) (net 4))
 (segment (start 69.93326 57) (end 74.6 57) (width 1) (layer F.Cu) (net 4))
 (segment (start 79.2 57) (end 80 56.2) (width 1) (layer F.Cu) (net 4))
 (segment (start 78.5 57) (end 79.2 57) (width 1) (layer F.Cu) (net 4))
 (segment (start 80 55) (end 80 51) (width 1) (layer F.Cu) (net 4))
 (segment (start 80 56.2) (end 80 55.5) (width 1) (layer F.Cu) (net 4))
 (segment (start 80 55.5) (end 80 55) (width 1) (layer F.Cu) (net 4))
 (segment (start 83.12 51) (end 80 51) (width 1) (layer F.Cu) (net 4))
 (segment (start 84.66 52.54) (end 83.12 51) (width 1) (layer F.Cu) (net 4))
 (segment (start 81.5 55.5) (end 80 55.5) (width 1) (layer F.Cu) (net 4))
 (segment (start 82.12 57.62) (end 82.12 56.12) (width 1) (layer F.Cu) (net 4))
 (segment (start 82.12 56.12) (end 81.5 55.5) (width 1) (layer F.Cu) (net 4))
 (segment (start 73.674999 54.716413) (end 73.674999 45.124999) (width 0.2) (layer F.Cu) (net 9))
 (segment (start 73.674999 45.124999) (end 73.175 44.625) (width 0.2) (layer F.Cu) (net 9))
 (segment (start 72.741402 55.65001) (end 73.674999 54.716413) (width 0.2) (layer F.Cu) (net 9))
 (segment (start 71.43501 55.65001) (end 72.741402 55.65001) (width 0.2) (layer F.Cu) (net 9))
 (segment (start 71.135 55.35) (end 71.43501 55.65001) (width 0.2) (layer F.Cu) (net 9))
 (segment (start 71.135 54.55) (end 71.135 55.35) (width 0.2) (layer F.Cu) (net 9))
 (segment (start 71.425 44.625) (end 70.875 44.625) (width 0.25) (layer F.Cu) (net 11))
 (segment (start 70.6 44.9) (end 70.0875 44.9) (width 0.25) (layer F.Cu) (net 11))
 (segment (start 70.875 44.625) (end 70.6 44.9) (width 0.25) (layer F.Cu) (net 11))
 (segment (start 75.05 46.25) (end 75.05 45.7375) (width 0.2) (layer F.Cu) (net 14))
 (segment (start 74.5 46.8) (end 75.05 46.25) (width 0.2) (layer F.Cu) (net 14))
 (segment (start 76.15 47.4) (end 76.15 48.13) (width 0.2) (layer F.Cu) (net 14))
 (segment (start 75.98 48.3) (end 74.704998 48.3) (width 0.2) (layer F.Cu) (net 14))
 (segment (start 74.704998 48.3) (end 74.5 48.095002) (width 0.2) (layer F.Cu) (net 14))
 (segment (start 76.15 48.13) (end 75.98 48.3) (width 0.2) (layer F.Cu) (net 14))
 (segment (start 74.5 48.095002) (end 74.5 46.8) (width 0.2) (layer F.Cu) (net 14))
 (segment (start 72.4 47.4875) (end 71.7125 47.4875) (width 0.25) (layer F.Cu) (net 12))
 (segment (start 71.135 48.065) (end 71.135 49.25) (width 0.25) (layer F.Cu) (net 12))
 (segment (start 71.7125 47.4875) (end 71.135 48.065) (width 0.25) (layer F.Cu) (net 12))
 (segment (start 76.439998 43.75) (end 77.1 43.75) (width 0.25) (layer F.Cu) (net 7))
 (segment (start 75.2 46.8) (end 75.455001 46.544999) (width 0.25) (layer F.Cu) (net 7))
 (segment (start 76.244999 46.205001) (end 76.244999 43.944999) (width 0.25) (layer F.Cu) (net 7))
 (segment (start 75.2 47.4) (end 75.2 46.8) (width 0.25) (layer F.Cu) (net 7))
 (segment (start 75.455001 46.544999) (end 75.905001 46.544999) (width 0.25) (layer F.Cu) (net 7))
 (segment (start 76.244999 43.944999) (end 76.439998 43.75) (width 0.25) (layer F.Cu) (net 7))
 (segment (start 75.905001 46.544999) (end 76.244999 46.205001) (width 0.25) (layer F.Cu) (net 7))
 (segment (start 77.1 47.4) (end 77.1 46.55) (width 0.25) (layer F.Cu) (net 6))
 (segment (start 77.1 46.55) (end 77.1 45.65) (width 0.25) (layer F.Cu) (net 6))
 (segment (start 79.3 44.7) (end 77.1 44.7) (width 0.25) (layer F.Cu) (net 5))
 (segment (start 74.075009 43.850009) (end 73.8 43.575) (width 0.2) (layer F.Cu) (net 8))
 (segment (start 72.907091 56.05002) (end 74.075009 54.882102) (width 0.2) (layer F.Cu) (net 8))
 (segment (start 70.56502 56.05002) (end 72.907091 56.05002) (width 0.2) (layer F.Cu) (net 8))
 (segment (start 74.075009 54.882102) (end 74.075009 43.850009) (width 0.2) (layer F.Cu) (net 8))
 (segment (start 69.865 55.35) (end 70.56502 56.05002) (width 0.2) (layer F.Cu) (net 8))
 (segment (start 73.8 43.575) (end 73.175 43.575) (width 0.2) (layer F.Cu) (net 8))
 (segment (start 69.865 54.55) (end 69.865 55.35) (width 0.2) (layer F.Cu) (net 8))
 (segment (start 71.425 43.575) (end 70.875 43.575) (width 0.25) (layer F.Cu) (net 10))
 (segment (start 70.6 43.3) (end 70.0875 43.3) (width 0.25) (layer F.Cu) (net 10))
 (segment (start 70.875 43.575) (end 70.6 43.3) (width 0.25) (layer F.Cu) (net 10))
 (segment (start 77.45 51.9875) (end 77.4375 52) (width 0.25) (layer F.Cu) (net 3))
 (segment (start 77.45 51.2) (end 77.45 51.9875) (width 0.25) (layer F.Cu) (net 3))
 (segment (start 77.1 49.6) (end 77.1 50.85) (width 0.25) (layer F.Cu) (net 3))
 (segment (start 77.1 50.85) (end 77.45 51.2) (width 0.25) (layer F.Cu) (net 3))
 (segment (start 77.1 49.6) (end 78.15 49.6) (width 0.25) (layer F.Cu) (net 3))
 (segment (start 78.15 49.6) (end 78.75 49) (width 0.25) (layer F.Cu) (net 3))
 (segment (start 78.75 49) (end 79.05 49) (width 0.25) (layer F.Cu) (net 3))
 (segment (start 79.3 45.65) (end 79.3 46) (width 0.5) (layer F.Cu) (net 3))
 (segment (start 79.3 46) (end 79.3 46.4) (width 1) (layer F.Cu) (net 3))
 (segment (start 79.05 49) (end 80 49) (width 0.25) (layer F.Cu) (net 3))
 (segment (start 80 47.1) (end 79.3 46.4) (width 1) (layer F.Cu) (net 3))
 (segment (start 80 49) (end 80 47.1) (width 1) (layer F.Cu) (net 3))
 (segment (start 81.75 49) (end 80 49) (width 1) (layer F.Cu) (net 3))
 (segment (start 84.66 47.46) (end 83.12 49) (width 1) (layer F.Cu) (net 3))
 (segment (start 83.12 49) (end 81.75 49) (width 1) (layer F.Cu) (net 3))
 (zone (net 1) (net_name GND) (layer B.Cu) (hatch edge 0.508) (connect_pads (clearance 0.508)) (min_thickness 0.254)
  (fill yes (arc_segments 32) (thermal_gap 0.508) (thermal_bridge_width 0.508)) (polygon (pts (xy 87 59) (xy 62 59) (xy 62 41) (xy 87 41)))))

